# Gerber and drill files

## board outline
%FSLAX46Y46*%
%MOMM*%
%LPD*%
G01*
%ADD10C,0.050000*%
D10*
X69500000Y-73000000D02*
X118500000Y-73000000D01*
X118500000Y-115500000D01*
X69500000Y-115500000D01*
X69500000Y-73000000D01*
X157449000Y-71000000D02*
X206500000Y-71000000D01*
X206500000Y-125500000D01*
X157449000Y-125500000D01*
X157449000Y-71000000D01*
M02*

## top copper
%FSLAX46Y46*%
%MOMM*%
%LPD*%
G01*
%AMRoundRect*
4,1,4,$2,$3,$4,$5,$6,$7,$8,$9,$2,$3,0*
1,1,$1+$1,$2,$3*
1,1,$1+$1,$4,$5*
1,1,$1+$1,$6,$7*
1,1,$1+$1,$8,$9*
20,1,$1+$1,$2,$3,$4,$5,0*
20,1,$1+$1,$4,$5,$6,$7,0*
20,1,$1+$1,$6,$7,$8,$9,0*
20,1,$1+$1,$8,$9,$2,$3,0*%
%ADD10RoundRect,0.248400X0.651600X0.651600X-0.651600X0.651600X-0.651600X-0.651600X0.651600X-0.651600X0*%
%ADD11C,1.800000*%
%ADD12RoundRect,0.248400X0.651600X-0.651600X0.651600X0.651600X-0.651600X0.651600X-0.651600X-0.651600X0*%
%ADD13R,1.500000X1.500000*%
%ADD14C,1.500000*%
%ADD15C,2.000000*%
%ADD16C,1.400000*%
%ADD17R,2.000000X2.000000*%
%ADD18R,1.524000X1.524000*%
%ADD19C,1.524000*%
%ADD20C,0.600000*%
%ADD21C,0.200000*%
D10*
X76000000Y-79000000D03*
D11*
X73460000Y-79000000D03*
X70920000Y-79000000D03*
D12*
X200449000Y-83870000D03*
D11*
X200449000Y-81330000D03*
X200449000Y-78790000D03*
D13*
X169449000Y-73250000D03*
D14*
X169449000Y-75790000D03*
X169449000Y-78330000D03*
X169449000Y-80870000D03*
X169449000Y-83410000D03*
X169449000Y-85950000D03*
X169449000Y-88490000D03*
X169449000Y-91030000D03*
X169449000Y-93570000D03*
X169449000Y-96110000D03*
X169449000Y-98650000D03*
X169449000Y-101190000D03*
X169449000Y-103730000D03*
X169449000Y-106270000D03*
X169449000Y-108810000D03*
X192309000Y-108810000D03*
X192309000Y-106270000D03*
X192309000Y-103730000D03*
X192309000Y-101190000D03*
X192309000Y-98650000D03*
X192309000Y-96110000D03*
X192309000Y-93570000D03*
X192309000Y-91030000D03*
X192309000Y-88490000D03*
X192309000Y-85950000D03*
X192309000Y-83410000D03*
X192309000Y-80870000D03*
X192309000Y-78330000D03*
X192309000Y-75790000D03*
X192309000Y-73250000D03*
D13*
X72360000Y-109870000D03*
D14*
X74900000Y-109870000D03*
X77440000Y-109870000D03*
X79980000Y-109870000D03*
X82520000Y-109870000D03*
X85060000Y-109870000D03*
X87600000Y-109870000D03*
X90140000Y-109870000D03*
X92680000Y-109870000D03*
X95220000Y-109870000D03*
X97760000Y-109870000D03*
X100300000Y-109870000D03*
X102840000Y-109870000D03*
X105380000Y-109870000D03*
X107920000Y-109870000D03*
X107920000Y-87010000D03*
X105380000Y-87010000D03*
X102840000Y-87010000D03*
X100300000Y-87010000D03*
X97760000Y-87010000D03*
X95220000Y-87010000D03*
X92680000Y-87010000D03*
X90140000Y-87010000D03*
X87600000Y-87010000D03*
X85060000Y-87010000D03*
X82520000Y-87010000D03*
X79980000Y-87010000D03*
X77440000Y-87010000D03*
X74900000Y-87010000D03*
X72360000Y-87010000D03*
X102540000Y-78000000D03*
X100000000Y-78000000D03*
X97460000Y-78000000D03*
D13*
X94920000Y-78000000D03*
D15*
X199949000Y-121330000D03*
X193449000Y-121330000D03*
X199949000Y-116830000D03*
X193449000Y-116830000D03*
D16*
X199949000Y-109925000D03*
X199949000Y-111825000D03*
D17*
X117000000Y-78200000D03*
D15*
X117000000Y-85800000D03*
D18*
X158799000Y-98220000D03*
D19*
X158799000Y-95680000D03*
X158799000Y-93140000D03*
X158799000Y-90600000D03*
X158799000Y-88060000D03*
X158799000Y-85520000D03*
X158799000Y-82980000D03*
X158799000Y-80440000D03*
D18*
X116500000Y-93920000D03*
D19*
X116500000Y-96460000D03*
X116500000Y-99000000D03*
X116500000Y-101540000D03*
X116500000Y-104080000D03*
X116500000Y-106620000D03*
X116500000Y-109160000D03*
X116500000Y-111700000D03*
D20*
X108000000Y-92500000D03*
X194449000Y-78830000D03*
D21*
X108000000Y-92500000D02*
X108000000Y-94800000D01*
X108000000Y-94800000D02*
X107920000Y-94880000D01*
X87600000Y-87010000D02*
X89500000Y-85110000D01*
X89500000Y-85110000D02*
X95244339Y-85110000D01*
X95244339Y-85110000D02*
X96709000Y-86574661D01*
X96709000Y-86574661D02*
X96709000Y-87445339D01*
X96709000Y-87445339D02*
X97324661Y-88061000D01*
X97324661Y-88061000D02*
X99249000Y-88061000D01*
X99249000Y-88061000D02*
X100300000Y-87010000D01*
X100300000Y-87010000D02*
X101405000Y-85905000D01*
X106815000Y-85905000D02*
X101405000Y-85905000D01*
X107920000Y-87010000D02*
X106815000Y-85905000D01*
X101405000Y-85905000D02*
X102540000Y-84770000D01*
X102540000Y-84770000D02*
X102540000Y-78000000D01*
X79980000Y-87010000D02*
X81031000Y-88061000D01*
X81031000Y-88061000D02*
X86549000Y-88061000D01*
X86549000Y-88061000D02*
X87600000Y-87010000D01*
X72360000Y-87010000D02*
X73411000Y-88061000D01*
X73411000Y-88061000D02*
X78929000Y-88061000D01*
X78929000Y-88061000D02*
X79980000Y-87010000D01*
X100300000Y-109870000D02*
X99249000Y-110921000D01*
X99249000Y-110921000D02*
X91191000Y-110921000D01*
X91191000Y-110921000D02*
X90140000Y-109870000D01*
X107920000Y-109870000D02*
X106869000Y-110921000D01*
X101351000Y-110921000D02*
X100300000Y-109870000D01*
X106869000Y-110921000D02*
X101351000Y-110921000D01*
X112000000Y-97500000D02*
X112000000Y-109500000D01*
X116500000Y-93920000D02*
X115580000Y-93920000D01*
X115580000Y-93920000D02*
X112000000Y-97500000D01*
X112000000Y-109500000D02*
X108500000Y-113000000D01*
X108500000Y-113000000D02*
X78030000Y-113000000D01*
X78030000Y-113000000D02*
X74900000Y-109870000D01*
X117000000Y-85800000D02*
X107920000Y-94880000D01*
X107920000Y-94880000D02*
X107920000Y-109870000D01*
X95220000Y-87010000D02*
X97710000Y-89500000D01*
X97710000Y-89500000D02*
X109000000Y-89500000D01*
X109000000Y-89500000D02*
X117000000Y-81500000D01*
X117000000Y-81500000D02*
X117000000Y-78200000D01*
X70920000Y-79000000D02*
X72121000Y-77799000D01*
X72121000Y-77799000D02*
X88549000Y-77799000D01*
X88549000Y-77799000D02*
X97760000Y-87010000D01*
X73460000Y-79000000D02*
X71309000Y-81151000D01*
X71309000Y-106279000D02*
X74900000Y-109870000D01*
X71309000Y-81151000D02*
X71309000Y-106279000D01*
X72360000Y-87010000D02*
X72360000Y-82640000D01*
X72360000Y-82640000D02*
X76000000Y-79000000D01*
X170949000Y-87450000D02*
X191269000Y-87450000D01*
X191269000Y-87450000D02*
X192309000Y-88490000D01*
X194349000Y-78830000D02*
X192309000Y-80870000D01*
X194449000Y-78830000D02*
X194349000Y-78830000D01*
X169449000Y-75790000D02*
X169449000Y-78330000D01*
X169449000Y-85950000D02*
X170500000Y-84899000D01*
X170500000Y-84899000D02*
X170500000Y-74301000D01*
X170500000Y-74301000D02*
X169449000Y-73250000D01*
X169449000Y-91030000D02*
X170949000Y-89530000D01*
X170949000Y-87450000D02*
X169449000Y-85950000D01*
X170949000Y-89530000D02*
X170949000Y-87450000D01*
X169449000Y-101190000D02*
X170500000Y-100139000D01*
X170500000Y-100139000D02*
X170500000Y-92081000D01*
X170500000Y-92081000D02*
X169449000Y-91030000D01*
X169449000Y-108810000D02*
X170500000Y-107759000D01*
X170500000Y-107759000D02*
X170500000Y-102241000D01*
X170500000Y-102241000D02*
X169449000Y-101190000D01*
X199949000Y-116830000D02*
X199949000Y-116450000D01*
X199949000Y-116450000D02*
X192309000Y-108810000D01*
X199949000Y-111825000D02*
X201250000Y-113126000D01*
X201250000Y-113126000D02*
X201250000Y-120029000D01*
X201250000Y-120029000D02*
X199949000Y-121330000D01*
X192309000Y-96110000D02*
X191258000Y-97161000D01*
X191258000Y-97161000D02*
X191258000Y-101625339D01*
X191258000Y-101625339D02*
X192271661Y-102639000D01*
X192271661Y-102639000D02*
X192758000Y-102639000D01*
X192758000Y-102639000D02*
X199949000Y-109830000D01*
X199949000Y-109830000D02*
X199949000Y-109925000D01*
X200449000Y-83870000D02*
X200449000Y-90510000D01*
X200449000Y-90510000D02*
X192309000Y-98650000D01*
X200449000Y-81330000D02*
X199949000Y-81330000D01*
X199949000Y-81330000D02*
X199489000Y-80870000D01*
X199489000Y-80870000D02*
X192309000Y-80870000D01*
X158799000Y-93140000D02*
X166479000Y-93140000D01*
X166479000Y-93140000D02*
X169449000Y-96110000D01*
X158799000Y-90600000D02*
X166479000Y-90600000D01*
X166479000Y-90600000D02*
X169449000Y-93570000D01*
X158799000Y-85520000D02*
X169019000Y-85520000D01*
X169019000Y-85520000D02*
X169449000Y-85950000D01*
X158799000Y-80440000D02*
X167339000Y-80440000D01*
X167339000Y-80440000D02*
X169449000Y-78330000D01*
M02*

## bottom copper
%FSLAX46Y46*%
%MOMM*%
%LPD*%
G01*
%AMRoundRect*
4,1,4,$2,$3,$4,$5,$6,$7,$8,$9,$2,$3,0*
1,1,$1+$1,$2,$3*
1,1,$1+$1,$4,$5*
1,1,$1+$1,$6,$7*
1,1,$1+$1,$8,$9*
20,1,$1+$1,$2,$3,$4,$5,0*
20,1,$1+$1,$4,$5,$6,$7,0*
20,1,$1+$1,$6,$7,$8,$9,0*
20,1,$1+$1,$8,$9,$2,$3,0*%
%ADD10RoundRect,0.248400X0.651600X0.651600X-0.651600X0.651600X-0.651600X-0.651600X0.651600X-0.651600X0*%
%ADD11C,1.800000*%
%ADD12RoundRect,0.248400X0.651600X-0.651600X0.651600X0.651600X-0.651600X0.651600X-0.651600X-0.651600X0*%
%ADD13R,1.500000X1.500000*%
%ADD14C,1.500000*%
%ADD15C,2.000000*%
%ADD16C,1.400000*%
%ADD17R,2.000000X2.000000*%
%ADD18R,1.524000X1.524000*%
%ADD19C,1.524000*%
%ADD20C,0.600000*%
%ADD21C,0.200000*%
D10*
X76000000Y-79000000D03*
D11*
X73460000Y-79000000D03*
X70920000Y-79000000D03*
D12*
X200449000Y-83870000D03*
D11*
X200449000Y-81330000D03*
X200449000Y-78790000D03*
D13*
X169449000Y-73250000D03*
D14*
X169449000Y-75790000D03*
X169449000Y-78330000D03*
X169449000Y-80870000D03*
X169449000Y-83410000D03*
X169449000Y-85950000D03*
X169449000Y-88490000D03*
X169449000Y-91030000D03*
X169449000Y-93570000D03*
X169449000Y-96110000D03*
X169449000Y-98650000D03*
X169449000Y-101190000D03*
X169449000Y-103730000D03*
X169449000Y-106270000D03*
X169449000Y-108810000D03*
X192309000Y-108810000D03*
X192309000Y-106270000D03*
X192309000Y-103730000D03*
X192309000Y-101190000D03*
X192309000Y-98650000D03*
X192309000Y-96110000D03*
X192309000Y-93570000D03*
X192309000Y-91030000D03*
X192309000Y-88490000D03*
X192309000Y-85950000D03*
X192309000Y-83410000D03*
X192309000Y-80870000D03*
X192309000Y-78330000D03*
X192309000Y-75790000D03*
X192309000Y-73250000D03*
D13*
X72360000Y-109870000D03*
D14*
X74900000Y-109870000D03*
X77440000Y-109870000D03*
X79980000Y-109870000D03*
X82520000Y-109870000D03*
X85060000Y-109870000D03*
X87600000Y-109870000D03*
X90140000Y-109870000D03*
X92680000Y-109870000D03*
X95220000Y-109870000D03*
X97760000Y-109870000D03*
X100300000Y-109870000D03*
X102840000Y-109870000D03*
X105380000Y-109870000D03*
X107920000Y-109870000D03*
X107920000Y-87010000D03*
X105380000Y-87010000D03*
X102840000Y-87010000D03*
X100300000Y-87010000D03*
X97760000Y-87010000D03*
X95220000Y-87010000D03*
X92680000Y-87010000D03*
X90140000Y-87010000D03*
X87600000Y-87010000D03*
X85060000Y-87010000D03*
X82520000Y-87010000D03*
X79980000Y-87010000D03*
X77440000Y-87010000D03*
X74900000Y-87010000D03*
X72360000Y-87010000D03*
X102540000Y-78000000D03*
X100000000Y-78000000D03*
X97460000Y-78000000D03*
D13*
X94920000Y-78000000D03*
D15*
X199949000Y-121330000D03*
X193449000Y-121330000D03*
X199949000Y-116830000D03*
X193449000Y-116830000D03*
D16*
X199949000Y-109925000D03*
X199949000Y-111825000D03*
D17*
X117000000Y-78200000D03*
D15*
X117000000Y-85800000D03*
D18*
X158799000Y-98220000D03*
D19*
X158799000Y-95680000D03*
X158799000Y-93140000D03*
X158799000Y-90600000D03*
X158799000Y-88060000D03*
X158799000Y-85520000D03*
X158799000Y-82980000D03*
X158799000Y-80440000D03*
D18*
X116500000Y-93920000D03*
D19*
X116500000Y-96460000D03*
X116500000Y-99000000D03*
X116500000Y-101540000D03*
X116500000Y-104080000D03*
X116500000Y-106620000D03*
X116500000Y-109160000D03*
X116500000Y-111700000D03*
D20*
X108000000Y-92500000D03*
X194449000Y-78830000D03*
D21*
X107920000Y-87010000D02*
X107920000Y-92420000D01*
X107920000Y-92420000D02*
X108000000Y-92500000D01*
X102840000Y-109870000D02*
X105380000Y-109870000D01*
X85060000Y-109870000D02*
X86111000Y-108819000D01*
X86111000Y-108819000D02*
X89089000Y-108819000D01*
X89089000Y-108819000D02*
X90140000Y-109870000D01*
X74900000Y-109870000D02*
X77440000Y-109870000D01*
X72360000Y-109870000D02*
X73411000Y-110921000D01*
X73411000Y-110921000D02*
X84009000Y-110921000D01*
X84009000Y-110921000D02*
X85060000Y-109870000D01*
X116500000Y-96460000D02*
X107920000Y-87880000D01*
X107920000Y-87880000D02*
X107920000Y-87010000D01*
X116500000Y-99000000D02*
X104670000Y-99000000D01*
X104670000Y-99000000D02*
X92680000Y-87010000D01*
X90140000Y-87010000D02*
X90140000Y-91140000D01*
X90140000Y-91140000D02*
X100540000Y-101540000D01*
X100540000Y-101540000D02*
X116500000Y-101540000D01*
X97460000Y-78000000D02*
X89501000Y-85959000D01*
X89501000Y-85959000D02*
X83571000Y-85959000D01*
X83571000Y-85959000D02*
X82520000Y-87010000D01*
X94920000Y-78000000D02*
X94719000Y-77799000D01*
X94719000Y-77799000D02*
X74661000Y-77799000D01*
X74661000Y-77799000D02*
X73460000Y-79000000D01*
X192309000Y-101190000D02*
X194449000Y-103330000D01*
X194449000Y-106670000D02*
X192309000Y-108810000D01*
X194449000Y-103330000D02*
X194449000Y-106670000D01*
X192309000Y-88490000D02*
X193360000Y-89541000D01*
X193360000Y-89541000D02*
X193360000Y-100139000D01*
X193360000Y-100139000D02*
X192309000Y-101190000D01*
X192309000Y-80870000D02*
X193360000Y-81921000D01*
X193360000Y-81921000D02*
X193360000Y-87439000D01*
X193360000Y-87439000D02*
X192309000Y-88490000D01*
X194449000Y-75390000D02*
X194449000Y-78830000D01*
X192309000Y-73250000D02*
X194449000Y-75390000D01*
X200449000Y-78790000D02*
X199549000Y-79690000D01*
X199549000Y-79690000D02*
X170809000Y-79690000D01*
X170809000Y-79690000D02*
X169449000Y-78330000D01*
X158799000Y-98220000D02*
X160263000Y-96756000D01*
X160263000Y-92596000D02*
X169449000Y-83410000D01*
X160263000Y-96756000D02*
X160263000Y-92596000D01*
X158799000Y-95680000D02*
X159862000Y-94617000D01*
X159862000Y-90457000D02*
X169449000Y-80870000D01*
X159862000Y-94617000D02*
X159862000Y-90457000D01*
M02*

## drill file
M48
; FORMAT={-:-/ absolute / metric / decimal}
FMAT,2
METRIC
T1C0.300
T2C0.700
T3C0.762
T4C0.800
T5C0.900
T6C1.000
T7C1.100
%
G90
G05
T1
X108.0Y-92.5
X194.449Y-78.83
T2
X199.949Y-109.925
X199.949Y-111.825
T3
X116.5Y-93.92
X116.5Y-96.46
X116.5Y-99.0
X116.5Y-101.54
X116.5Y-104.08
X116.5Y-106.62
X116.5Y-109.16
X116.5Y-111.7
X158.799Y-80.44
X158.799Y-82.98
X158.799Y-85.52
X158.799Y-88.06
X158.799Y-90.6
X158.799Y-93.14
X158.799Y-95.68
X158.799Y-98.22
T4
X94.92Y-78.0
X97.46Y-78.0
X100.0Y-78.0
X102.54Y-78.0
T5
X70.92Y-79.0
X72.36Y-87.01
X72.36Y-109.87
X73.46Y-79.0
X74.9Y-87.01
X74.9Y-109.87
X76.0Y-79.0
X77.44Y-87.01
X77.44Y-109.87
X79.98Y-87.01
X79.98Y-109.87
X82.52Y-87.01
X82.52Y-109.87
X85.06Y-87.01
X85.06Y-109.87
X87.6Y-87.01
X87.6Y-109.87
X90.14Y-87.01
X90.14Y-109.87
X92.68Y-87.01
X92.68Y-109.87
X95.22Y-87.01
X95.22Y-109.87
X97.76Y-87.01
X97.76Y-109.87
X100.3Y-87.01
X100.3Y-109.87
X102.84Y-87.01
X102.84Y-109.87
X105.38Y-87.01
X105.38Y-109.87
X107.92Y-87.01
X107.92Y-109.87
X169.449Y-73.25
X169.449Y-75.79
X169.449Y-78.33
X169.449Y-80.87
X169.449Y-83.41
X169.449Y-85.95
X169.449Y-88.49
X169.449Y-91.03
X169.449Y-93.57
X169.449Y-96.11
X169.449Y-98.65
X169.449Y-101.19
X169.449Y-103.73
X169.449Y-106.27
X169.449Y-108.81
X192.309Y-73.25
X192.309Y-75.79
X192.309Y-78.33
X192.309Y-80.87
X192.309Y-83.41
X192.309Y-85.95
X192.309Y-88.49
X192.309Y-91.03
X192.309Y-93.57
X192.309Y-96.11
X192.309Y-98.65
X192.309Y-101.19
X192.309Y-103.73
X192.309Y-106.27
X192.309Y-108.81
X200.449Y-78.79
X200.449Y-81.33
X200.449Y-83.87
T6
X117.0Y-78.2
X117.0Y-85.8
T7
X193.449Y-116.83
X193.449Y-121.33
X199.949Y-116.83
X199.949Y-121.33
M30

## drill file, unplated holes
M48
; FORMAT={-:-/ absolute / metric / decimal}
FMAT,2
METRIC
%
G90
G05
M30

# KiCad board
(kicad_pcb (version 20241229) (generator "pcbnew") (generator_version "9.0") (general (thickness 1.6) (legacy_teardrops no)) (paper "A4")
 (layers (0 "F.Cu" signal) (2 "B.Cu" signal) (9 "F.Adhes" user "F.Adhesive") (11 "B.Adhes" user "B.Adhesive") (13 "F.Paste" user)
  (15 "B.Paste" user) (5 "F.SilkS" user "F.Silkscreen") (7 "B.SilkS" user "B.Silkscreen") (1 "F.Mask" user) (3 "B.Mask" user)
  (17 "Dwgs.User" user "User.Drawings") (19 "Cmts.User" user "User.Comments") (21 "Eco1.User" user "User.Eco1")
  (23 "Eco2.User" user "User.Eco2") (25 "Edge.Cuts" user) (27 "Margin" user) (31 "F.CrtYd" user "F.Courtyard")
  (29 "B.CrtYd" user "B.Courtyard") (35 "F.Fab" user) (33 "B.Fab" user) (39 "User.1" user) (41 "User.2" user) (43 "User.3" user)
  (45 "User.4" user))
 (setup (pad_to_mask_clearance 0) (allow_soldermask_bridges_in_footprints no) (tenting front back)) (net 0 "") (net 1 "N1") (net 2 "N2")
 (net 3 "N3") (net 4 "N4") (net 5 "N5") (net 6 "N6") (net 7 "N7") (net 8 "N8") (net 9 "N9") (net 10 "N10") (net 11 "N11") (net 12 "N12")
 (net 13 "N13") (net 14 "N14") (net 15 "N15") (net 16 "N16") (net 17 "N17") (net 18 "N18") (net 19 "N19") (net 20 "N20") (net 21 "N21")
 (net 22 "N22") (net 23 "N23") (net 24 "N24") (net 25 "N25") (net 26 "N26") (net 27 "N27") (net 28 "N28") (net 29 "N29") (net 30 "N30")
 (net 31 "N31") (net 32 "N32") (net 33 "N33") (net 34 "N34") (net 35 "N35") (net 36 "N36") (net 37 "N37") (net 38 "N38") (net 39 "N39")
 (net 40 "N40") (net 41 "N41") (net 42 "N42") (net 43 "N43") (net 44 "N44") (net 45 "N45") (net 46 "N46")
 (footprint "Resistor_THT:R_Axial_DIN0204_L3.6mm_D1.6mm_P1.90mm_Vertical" (layer "F.Cu") (at 199.949 109.925 -90)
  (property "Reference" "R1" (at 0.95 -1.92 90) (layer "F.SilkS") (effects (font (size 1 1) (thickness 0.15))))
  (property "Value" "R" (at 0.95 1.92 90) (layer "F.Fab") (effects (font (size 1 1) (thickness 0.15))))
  (pad "1" thru_hole circle (at 0 0 270) (size 1.4 1.4) (drill 0.7) (layers "*.Cu" "*.Mask") (remove_unused_layers no) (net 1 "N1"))
  (pad "2" thru_hole circle (at 1.9 0 270) (size 1.4 1.4) (drill 0.7) (layers "*.Cu" "*.Mask") (remove_unused_layers no) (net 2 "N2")))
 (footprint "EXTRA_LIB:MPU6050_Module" (layer "F.Cu") (at 116.5 93.92)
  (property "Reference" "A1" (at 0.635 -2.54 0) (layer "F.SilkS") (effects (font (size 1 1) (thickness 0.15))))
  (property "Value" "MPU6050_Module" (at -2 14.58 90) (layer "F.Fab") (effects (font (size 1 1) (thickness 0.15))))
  (pad "1" thru_hole rect (at 0 0) (size 1.524 1.524) (drill 0.762) (layers "*.Cu" "*.Mask") (remove_unused_layers no) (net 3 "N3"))
  (pad "2" thru_hole circle (at 0 2.54) (size 1.524 1.524) (drill 0.762) (layers "*.Cu" "*.Mask") (remove_unused_layers no) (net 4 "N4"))
  (pad "3" thru_hole circle (at 0 5.08) (size 1.524 1.524) (drill 0.762) (layers "*.Cu" "*.Mask") (remove_unused_layers no) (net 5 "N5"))
  (pad "4" thru_hole circle (at 0 7.62) (size 1.524 1.524) (drill 0.762) (layers "*.Cu" "*.Mask") (remove_unused_layers no) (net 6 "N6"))
  (pad "5" thru_hole circle (at 0 10.16) (size 1.524 1.524) (drill 0.762) (layers "*.Cu" "*.Mask") (remove_unused_layers no) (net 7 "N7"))
  (pad "6" thru_hole circle (at 0 12.7) (size 1.524 1.524) (drill 0.762) (layers "*.Cu" "*.Mask") (remove_unused_layers no) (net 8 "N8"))
  (pad "7" thru_hole circle (at 0 15.24) (size 1.524 1.524) (drill 0.762) (layers "*.Cu" "*.Mask") (remove_unused_layers no) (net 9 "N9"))
  (pad "8" thru_hole circle (at 0 17.78) (size 1.524 1.524) (drill 0.762) (layers "*.Cu" "*.Mask") (remove_unused_layers no) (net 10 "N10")))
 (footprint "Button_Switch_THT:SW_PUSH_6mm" (layer "F.Cu") (at 199.949 121.33 180)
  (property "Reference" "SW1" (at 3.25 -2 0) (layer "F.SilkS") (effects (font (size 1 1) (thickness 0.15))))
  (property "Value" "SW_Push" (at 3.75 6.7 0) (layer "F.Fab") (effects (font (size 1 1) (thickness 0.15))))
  (pad "1" thru_hole circle (at 0 0 270) (size 2 2) (drill 1.1) (layers "*.Cu" "*.Mask") (remove_unused_layers no) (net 2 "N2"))
  (pad "1" thru_hole circle (at 6.5 0 270) (size 2 2) (drill 1.1) (layers "*.Cu" "*.Mask") (remove_unused_layers no) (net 2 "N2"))
  (pad "2" thru_hole circle (at 0 4.5 270) (size 2 2) (drill 1.1) (layers "*.Cu" "*.Mask") (remove_unused_layers no) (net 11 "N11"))
  (pad "2" thru_hole circle (at 6.5 4.5 270) (size 2 2) (drill 1.1) (layers "*.Cu" "*.Mask") (remove_unused_layers no) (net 11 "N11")))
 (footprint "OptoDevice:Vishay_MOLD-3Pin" (layer "F.Cu") (at 200.449 83.87 90)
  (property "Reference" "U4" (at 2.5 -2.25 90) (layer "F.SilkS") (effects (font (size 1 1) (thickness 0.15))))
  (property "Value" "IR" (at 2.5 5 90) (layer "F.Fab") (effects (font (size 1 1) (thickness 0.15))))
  (pad "1" thru_hole roundrect (at 0 0 90) (size 1.8 1.8) (drill 0.9) (layers "*.Cu" "*.Mask") (remove_unused_layers no)
   (roundrect_rratio 0.138) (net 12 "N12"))
  (pad "2" thru_hole circle (at 2.54 0 90) (size 1.8 1.8) (drill 0.9) (layers "*.Cu" "*.Mask") (remove_unused_layers no) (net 11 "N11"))
  (pad "3" thru_hole circle (at 5.08 0 90) (size 1.8 1.8) (drill 0.9) (layers "*.Cu" "*.Mask") (remove_unused_layers no) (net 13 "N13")))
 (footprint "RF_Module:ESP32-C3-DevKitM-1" (layer "F.Cu") (at 72.36 109.87 90)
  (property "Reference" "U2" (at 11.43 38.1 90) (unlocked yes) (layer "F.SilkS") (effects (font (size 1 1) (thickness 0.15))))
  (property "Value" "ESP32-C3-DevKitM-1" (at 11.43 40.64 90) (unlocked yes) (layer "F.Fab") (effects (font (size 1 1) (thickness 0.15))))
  (pad "1" thru_hole rect (at 0 0 90) (size 1.5 1.5) (drill 0.9) (layers "*.Cu" "*.Mask") (remove_unused_layers yes) (keep_end_layers yes)
   (zone_layer_connections) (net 4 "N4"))
  (pad "2" thru_hole circle (at 0 2.54 90) (size 1.5 1.5) (drill 0.9) (layers "*.Cu" "*.Mask") (remove_unused_layers yes)
   (keep_end_layers yes) (zone_layer_connections) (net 3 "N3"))
  (pad "3" thru_hole circle (at 0 5.08 90) (size 1.5 1.5) (drill 0.9) (layers "*.Cu" "*.Mask") (remove_unused_layers yes)
   (keep_end_layers yes) (zone_layer_connections) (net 3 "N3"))
  (pad "4" thru_hole circle (at 0 7.62 90) (size 1.5 1.5) (drill 0.9) (layers "*.Cu" "*.Mask") (remove_unused_layers yes)
   (keep_end_layers yes) (zone_layer_connections) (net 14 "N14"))
  (pad "5" thru_hole circle (at 0 10.16 90) (size 1.5 1.5) (drill 0.9) (layers "*.Cu" "*.Mask") (remove_unused_layers yes)
   (keep_end_layers yes) (zone_layer_connections) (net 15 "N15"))
  (pad "6" thru_hole circle (at 0 12.7 90) (size 1.5 1.5) (drill 0.9) (layers "*.Cu" "*.Mask") (remove_unused_layers yes)
   (keep_end_layers yes) (zone_layer_connections) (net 4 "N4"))
  (pad "7" thru_hole circle (at 0 15.24 90) (size 1.5 1.5) (drill 0.9) (layers "*.Cu" "*.Mask") (remove_unused_layers yes)
   (keep_end_layers yes) (zone_layer_connections) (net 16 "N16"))
  (pad "8" thru_hole circle (at 0 17.78 90) (size 1.5 1.5) (drill 0.9) (layers "*.Cu" "*.Mask") (remove_unused_layers yes)
   (keep_end_layers yes) (zone_layer_connections) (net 4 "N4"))
  (pad "9" thru_hole circle (at 0 20.32 90) (size 1.5 1.5) (drill 0.9) (layers "*.Cu" "*.Mask") (remove_unused_layers yes)
   (keep_end_layers yes) (zone_layer_connections) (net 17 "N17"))
  (pad "10" thru_hole circle (at 0 22.86 90) (size 1.5 1.5) (drill 0.9) (layers "*.Cu" "*.Mask") (remove_unused_layers yes)
   (keep_end_layers yes) (zone_layer_connections) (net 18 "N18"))
  (pad "11" thru_hole circle (at 0 25.4 90) (size 1.5 1.5) (drill 0.9) (layers "*.Cu" "*.Mask") (remove_unused_layers yes)
   (keep_end_layers yes) (zone_layer_connections) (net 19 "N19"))
  (pad "12" thru_hole circle (at 0 27.94 90) (size 1.5 1.5) (drill 0.9) (layers "*.Cu" "*.Mask") (remove_unused_layers yes)
   (keep_end_layers yes) (zone_layer_connections) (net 4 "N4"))
  (pad "13" thru_hole circle (at 0 30.48 90) (size 1.5 1.5) (drill 0.9) (layers "*.Cu" "*.Mask") (remove_unused_layers yes)
   (keep_end_layers yes) (zone_layer_connections) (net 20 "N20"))
  (pad "14" thru_hole circle (at 0 33.02 90) (size 1.5 1.5) (drill 0.9) (layers "*.Cu" "*.Mask") (remove_unused_layers yes)
   (keep_end_layers yes) (zone_layer_connections) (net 20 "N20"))
  (pad "15" thru_hole circle (at 0 35.56 90) (size 1.5 1.5) (drill 0.9) (layers "*.Cu" "*.Mask") (remove_unused_layers yes)
   (keep_end_layers yes) (zone_layer_connections) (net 4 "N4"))
  (pad "16" thru_hole circle (at 22.86 35.56 90) (size 1.5 1.5) (drill 0.9) (layers "*.Cu" "*.Mask") (remove_unused_layers yes)
   (keep_end_layers yes) (zone_layer_connections) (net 4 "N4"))
  (pad "17" thru_hole circle (at 22.86 33.02 90) (size 1.5 1.5) (drill 0.9) (layers "*.Cu" "*.Mask") (remove_unused_layers yes)
   (keep_end_layers yes) (zone_layer_connections) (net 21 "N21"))
  (pad "18" thru_hole circle (at 22.86 30.48 90) (size 1.5 1.5) (drill 0.9) (layers "*.Cu" "*.Mask") (remove_unused_layers yes)
   (keep_end_layers yes) (zone_layer_connections) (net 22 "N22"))
  (pad "19" thru_hole circle (at 22.86 27.94 90) (size 1.5 1.5) (drill 0.9) (layers "*.Cu" "*.Mask") (remove_unused_layers yes)
   (keep_end_layers yes) (zone_layer_connections) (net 4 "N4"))
  (pad "20" thru_hole circle (at 22.86 25.4 90) (size 1.5 1.5) (drill 0.9) (layers "*.Cu" "*.Mask") (remove_unused_layers yes)
   (keep_end_layers yes) (zone_layer_connections) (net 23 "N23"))
  (pad "21" thru_hole circle (at 22.86 22.86 90) (size 1.5 1.5) (drill 0.9) (layers "*.Cu" "*.Mask") (remove_unused_layers yes)
   (keep_end_layers yes) (zone_layer_connections) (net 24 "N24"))
  (pad "22" thru_hole circle (at 22.86 20.32 90) (size 1.5 1.5) (drill 0.9) (layers "*.Cu" "*.Mask") (remove_unused_layers yes)
   (keep_end_layers yes) (zone_layer_connections) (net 5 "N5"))
  (pad "23" thru_hole circle (at 22.86 17.78 90) (size 1.5 1.5) (drill 0.9) (layers "*.Cu" "*.Mask") (remove_unused_layers yes)
   (keep_end_layers yes) (zone_layer_connections) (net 6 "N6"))
  (pad "24" thru_hole circle (at 22.86 15.24 90) (size 1.5 1.5) (drill 0.9) (layers "*.Cu" "*.Mask") (remove_unused_layers yes)
   (keep_end_layers yes) (zone_layer_connections) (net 4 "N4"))
  (pad "25" thru_hole circle (at 22.86 12.7 90) (size 1.5 1.5) (drill 0.9) (layers "*.Cu" "*.Mask") (remove_unused_layers yes)
   (keep_end_layers yes) (zone_layer_connections) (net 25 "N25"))
  (pad "26" thru_hole circle (at 22.86 10.16 90) (size 1.5 1.5) (drill 0.9) (layers "*.Cu" "*.Mask") (remove_unused_layers yes)
   (keep_end_layers yes) (zone_layer_connections) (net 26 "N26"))
  (pad "27" thru_hole circle (at 22.86 7.62 90) (size 1.5 1.5) (drill 0.9) (layers "*.Cu" "*.Mask") (remove_unused_layers yes)
   (keep_end_layers yes) (zone_layer_connections) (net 4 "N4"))
  (pad "28" thru_hole circle (at 22.86 5.08 90) (size 1.5 1.5) (drill 0.9) (layers "*.Cu" "*.Mask") (remove_unused_layers yes)
   (keep_end_layers yes) (zone_layer_connections) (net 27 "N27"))
  (pad "29" thru_hole circle (at 22.86 2.54 90) (size 1.5 1.5) (drill 0.9) (layers "*.Cu" "*.Mask") (remove_unused_layers yes)
   (keep_end_layers yes) (zone_layer_connections) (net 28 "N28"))
  (pad "30" thru_hole circle (at 22.86 0 90) (size 1.5 1.5) (drill 0.9) (layers "*.Cu" "*.Mask") (remove_unused_layers yes)
   (keep_end_layers yes) (zone_layer_connections) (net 4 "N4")))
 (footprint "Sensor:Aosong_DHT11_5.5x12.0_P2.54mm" (layer "F.Cu") (at 94.92 78 90)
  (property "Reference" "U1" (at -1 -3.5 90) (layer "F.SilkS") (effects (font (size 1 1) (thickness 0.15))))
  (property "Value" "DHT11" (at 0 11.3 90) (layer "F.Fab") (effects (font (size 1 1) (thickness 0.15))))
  (pad "1" thru_hole rect (at 0 0 90) (size 1.5 1.5) (drill 0.8) (layers "*.Cu" "*.Mask") (remove_unused_layers no) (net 3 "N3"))
  (pad "2" thru_hole circle (at 0 2.54 90) (size 1.5 1.5) (drill 0.8) (layers "*.Cu" "*.Mask") (remove_unused_layers no) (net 26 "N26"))
  (pad "3" thru_hole circle (at 0 5.08 90) (size 1.5 1.5) (drill 0.8) (layers "*.Cu" "*.Mask") (remove_unused_layers no) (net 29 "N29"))
  (pad "4" thru_hole circle (at 0 7.62 90) (size 1.5 1.5) (drill 0.8) (layers "*.Cu" "*.Mask") (remove_unused_layers no) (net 4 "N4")))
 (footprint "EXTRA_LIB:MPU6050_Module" (layer "F.Cu") (at 158.799 98.22 180)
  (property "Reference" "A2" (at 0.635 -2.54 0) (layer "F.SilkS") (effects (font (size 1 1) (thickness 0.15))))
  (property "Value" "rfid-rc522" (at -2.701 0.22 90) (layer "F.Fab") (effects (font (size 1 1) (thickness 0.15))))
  (pad "1" thru_hole rect (at 0 0 180) (size 1.524 1.524) (drill 0.762) (layers "*.Cu" "*.Mask") (remove_unused_layers no) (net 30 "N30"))
  (pad "2" thru_hole circle (at 0 2.54 180) (size 1.524 1.524) (drill 0.762) (layers "*.Cu" "*.Mask") (remove_unused_layers no)
   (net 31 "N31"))
  (pad "3" thru_hole circle (at 0 5.08 180) (size 1.524 1.524) (drill 0.762) (layers "*.Cu" "*.Mask") (remove_unused_layers no)
   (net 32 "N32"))
  (pad "4" thru_hole circle (at 0 7.62 180) (size 1.524 1.524) (drill 0.762) (layers "*.Cu" "*.Mask") (remove_unused_layers no)
   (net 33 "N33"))
  (pad "5" thru_hole circle (at 0 10.16 180) (size 1.524 1.524) (drill 0.762) (layers "*.Cu" "*.Mask") (remove_unused_layers no)
   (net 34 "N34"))
  (pad "6" thru_hole circle (at 0 12.7 180) (size 1.524 1.524) (drill 0.762) (layers "*.Cu" "*.Mask") (remove_unused_layers no)
   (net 11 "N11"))
  (pad "7" thru_hole circle (at 0 15.24 180) (size 1.524 1.524) (drill 0.762) (layers "*.Cu" "*.Mask") (remove_unused_layers no)
   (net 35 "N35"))
  (pad "8" thru_hole circle (at 0 17.78 180) (size 1.524 1.524) (drill 0.762) (layers "*.Cu" "*.Mask") (remove_unused_layers no)
   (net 13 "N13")))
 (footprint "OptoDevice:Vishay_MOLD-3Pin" (layer "F.Cu") (at 76 79 180)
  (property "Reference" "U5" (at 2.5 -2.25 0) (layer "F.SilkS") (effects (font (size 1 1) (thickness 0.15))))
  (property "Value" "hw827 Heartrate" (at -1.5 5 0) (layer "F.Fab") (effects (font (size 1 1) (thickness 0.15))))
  (pad "1" thru_hole roundrect (at 0 0 180) (size 1.8 1.8) (drill 0.9) (layers "*.Cu" "*.Mask") (remove_unused_layers no)
   (roundrect_rratio 0.138) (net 4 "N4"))
  (pad "2" thru_hole circle (at 2.54 0 180) (size 1.8 1.8) (drill 0.9) (layers "*.Cu" "*.Mask") (remove_unused_layers no) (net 3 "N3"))
  (pad "3" thru_hole circle (at 5.08 0 180) (size 1.8 1.8) (drill 0.9) (layers "*.Cu" "*.Mask") (remove_unused_layers no) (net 23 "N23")))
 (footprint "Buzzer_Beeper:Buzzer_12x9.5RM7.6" (layer "F.Cu") (at 117 78.2 -90)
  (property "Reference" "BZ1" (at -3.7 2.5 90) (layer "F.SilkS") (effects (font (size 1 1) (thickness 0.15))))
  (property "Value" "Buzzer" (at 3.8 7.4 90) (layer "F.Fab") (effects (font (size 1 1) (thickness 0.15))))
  (pad "1" thru_hole rect (at 0 0 270) (size 2 2) (drill 1) (layers "*.Cu" "*.Mask") (remove_unused_layers no) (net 24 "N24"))
  (pad "2" thru_hole circle (at 7.6 0 270) (size 2 2) (drill 1) (layers "*.Cu" "*.Mask") (remove_unused_layers no) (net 4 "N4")))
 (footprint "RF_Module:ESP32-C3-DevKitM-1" (layer "F.Cu") (at 169.449 73.25)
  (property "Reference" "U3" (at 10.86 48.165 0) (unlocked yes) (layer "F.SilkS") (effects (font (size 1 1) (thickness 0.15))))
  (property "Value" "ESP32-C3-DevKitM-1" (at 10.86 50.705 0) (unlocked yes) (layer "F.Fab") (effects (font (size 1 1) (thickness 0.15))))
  (pad "1" thru_hole rect (at 0 0) (size 1.5 1.5) (drill 0.9) (layers "*.Cu" "*.Mask") (remove_unused_layers yes) (keep_end_layers yes)
   (zone_layer_connections) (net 11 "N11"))
  (pad "2" thru_hole circle (at 0 2.54) (size 1.5 1.5) (drill 0.9) (layers "*.Cu" "*.Mask") (remove_unused_layers yes) (keep_end_layers yes)
   (zone_layer_connections) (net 13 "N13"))
  (pad "3" thru_hole circle (at 0 5.08) (size 1.5 1.5) (drill 0.9) (layers "*.Cu" "*.Mask") (remove_unused_layers yes) (keep_end_layers yes)
   (zone_layer_connections) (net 13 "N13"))
  (pad "4" thru_hole circle (at 0 7.62) (size 1.5 1.5) (drill 0.9) (layers "*.Cu" "*.Mask") (remove_unused_layers yes) (keep_end_layers yes)
   (zone_layer_connections) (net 31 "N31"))
  (pad "5" thru_hole circle (at 0 10.16) (size 1.5 1.5) (drill 0.9) (layers "*.Cu" "*.Mask") (remove_unused_layers yes)
   (keep_end_layers yes) (zone_layer_connections) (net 30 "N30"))
  (pad "6" thru_hole circle (at 0 12.7) (size 1.5 1.5) (drill 0.9) (layers "*.Cu" "*.Mask") (remove_unused_layers yes) (keep_end_layers yes)
   (zone_layer_connections) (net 11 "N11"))
  (pad "7" thru_hole circle (at 0 15.24) (size 1.5 1.5) (drill 0.9) (layers "*.Cu" "*.Mask") (remove_unused_layers yes)
   (keep_end_layers yes) (zone_layer_connections) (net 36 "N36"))
  (pad "8" thru_hole circle (at 0 17.78) (size 1.5 1.5) (drill 0.9) (layers "*.Cu" "*.Mask") (remove_unused_layers yes)
   (keep_end_layers yes) (zone_layer_connections) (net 11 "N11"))
  (pad "9" thru_hole circle (at 0 20.32) (size 1.5 1.5) (drill 0.9) (layers "*.Cu" "*.Mask") (remove_unused_layers yes)
   (keep_end_layers yes) (zone_layer_connections) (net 33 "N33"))
  (pad "10" thru_hole circle (at 0 22.86) (size 1.5 1.5) (drill 0.9) (layers "*.Cu" "*.Mask") (remove_unused_layers yes)
   (keep_end_layers yes) (zone_layer_connections) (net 32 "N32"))
  (pad "11" thru_hole circle (at 0 25.4) (size 1.5 1.5) (drill 0.9) (layers "*.Cu" "*.Mask") (remove_unused_layers yes)
   (keep_end_layers yes) (zone_layer_connections) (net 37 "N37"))
  (pad "12" thru_hole circle (at 0 27.94) (size 1.5 1.5) (drill 0.9) (layers "*.Cu" "*.Mask") (remove_unused_layers yes)
   (keep_end_layers yes) (zone_layer_connections) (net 11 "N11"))
  (pad "13" thru_hole circle (at 0 30.48) (size 1.5 1.5) (drill 0.9) (layers "*.Cu" "*.Mask") (remove_unused_layers yes)
   (keep_end_layers yes) (zone_layer_connections) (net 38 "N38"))
  (pad "14" thru_hole circle (at 0 33.02) (size 1.5 1.5) (drill 0.9) (layers "*.Cu" "*.Mask") (remove_unused_layers yes)
   (keep_end_layers yes) (zone_layer_connections) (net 38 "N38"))
  (pad "15" thru_hole circle (at 0 35.56) (size 1.5 1.5) (drill 0.9) (layers "*.Cu" "*.Mask") (remove_unused_layers yes)
   (keep_end_layers yes) (zone_layer_connections) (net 11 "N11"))
  (pad "16" thru_hole circle (at 22.86 35.56) (size 1.5 1.5) (drill 0.9) (layers "*.Cu" "*.Mask") (remove_unused_layers yes)
   (keep_end_layers yes) (zone_layer_connections) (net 11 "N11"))
  (pad "17" thru_hole circle (at 22.86 33.02) (size 1.5 1.5) (drill 0.9) (layers "*.Cu" "*.Mask") (remove_unused_layers yes)
   (keep_end_layers yes) (zone_layer_connections) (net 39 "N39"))
  (pad "18" thru_hole circle (at 22.86 30.48) (size 1.5 1.5) (drill 0.9) (layers "*.Cu" "*.Mask") (remove_unused_layers yes)
   (keep_end_layers yes) (zone_layer_connections) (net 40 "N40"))
  (pad "19" thru_hole circle (at 22.86 27.94) (size 1.5 1.5) (drill 0.9) (layers "*.Cu" "*.Mask") (remove_unused_layers yes)
   (keep_end_layers yes) (zone_layer_connections) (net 11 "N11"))
  (pad "20" thru_hole circle (at 22.86 25.4) (size 1.5 1.5) (drill 0.9) (layers "*.Cu" "*.Mask") (remove_unused_layers yes)
   (keep_end_layers yes) (zone_layer_connections) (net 12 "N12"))
  (pad "21" thru_hole circle (at 22.86 22.86) (size 1.5 1.5) (drill 0.9) (layers "*.Cu" "*.Mask") (remove_unused_layers yes)
   (keep_end_layers yes) (zone_layer_connections) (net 1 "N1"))
  (pad "22" thru_hole circle (at 22.86 20.32) (size 1.5 1.5) (drill 0.9) (layers "*.Cu" "*.Mask") (remove_unused_layers yes)
   (keep_end_layers yes) (zone_layer_connections) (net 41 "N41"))
  (pad "23" thru_hole circle (at 22.86 17.78) (size 1.5 1.5) (drill 0.9) (layers "*.Cu" "*.Mask") (remove_unused_layers yes)
   (keep_end_layers yes) (zone_layer_connections) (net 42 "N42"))
  (pad "24" thru_hole circle (at 22.86 15.24) (size 1.5 1.5) (drill 0.9) (layers "*.Cu" "*.Mask") (remove_unused_layers yes)
   (keep_end_layers yes) (zone_layer_connections) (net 11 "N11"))
  (pad "25" thru_hole circle (at 22.86 12.7) (size 1.5 1.5) (drill 0.9) (layers "*.Cu" "*.Mask") (remove_unused_layers yes)
   (keep_end_layers yes) (zone_layer_connections) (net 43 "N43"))
  (pad "26" thru_hole circle (at 22.86 10.16) (size 1.5 1.5) (drill 0.9) (layers "*.Cu" "*.Mask") (remove_unused_layers yes)
   (keep_end_layers yes) (zone_layer_connections) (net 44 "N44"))
  (pad "27" thru_hole circle (at 22.86 7.62) (size 1.5 1.5) (drill 0.9) (layers "*.Cu" "*.Mask") (remove_unused_layers yes)
   (keep_end_layers yes) (zone_layer_connections) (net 11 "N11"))
  (pad "28" thru_hole circle (at 22.86 5.08) (size 1.5 1.5) (drill 0.9) (layers "*.Cu" "*.Mask") (remove_unused_layers yes)
   (keep_end_layers yes) (zone_layer_connections) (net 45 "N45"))
  (pad "29" thru_hole circle (at 22.86 2.54) (size 1.5 1.5) (drill 0.9) (layers "*.Cu" "*.Mask") (remove_unused_layers yes)
   (keep_end_layers yes) (zone_layer_connections) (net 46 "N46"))
  (pad "30" thru_hole circle (at 22.86 0) (size 1.5 1.5) (drill 0.9) (layers "*.Cu" "*.Mask") (remove_unused_layers yes)
   (keep_end_layers yes) (zone_layer_connections) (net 11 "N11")))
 (gr_rect (start 69.5 73) (end 118.5 115.5) (stroke (width 0.05) (type default)) (fill no) (layer "Edge.Cuts"))
 (gr_rect (start 157.449 71) (end 206.5 125.5) (stroke (width 0.05) (type default)) (fill no) (layer "Edge.Cuts"))
 (segment (start 71.309 106.279) (end 74.9 109.87) (width 0.2) (layer "F.Cu") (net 3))
 (segment (start 112 109.5) (end 108.5 113) (width 0.2) (layer "F.Cu") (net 3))
 (segment (start 116.5 93.92) (end 115.58 93.92) (width 0.2) (layer "F.Cu") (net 3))
 (segment (start 112 97.5) (end 112 109.5) (width 0.2) (layer "F.Cu") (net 3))
 (segment (start 115.58 93.92) (end 112 97.5) (width 0.2) (layer "F.Cu") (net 3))
 (segment (start 73.46 79) (end 71.309 81.151) (width 0.2) (layer "F.Cu") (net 3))
 (segment (start 108.5 113) (end 78.03 113) (width 0.2) (layer "F.Cu") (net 3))
 (segment (start 71.309 81.151) (end 71.309 106.279) (width 0.2) (layer "F.Cu") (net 3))
 (segment (start 78.03 113) (end 74.9 109.87) (width 0.2) (layer "F.Cu") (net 3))
 (segment (start 94.92 78) (end 94.719 77.799) (width 0.2) (layer "B.Cu") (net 3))
 (segment (start 94.719 77.799) (end 74.661 77.799) (width 0.2) (layer "B.Cu") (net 3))
 (segment (start 74.661 77.799) (end 73.46 79) (width 0.2) (layer "B.Cu") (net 3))
 (segment (start 74.9 109.87) (end 77.44 109.87) (width 0.2) (layer "B.Cu") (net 3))
 (segment (start 90.14 91.14) (end 100.54 101.54) (width 0.2) (layer "B.Cu") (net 6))
 (segment (start 100.54 101.54) (end 116.5 101.54) (width 0.2) (layer "B.Cu") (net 6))
 (segment (start 90.14 87.01) (end 90.14 91.14) (width 0.2) (layer "B.Cu") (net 6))
 (segment (start 73.411 88.061) (end 78.929 88.061) (width 0.2) (layer "F.Cu") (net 4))
 (segment (start 99.249 88.061) (end 100.3 87.01) (width 0.2) (layer "F.Cu") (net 4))
 (segment (start 72.36 87.01) (end 72.36 82.64) (width 0.2) (layer "F.Cu") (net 4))
 (segment (start 107.92 87.01) (end 106.815 85.905) (width 0.2) (layer "F.Cu") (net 4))
 (segment (start 96.709 87.445339) (end 97.324661 88.061) (width 0.2) (layer "F.Cu") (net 4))
 (segment (start 72.36 82.64) (end 76 79) (width 0.2) (layer "F.Cu") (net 4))
 (segment (start 107.92 109.87) (end 106.869 110.921) (width 0.2) (layer "F.Cu") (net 4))
 (segment (start 100.3 87.01) (end 101.405 85.905) (width 0.2) (layer "F.Cu") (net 4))
 (segment (start 97.324661 88.061) (end 99.249 88.061) (width 0.2) (layer "F.Cu") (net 4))
 (segment (start 81.031 88.061) (end 86.549 88.061) (width 0.2) (layer "F.Cu") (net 4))
 (segment (start 96.709 86.574661) (end 96.709 87.445339) (width 0.2) (layer "F.Cu") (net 4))
 (segment (start 106.869 110.921) (end 101.351 110.921) (width 0.2) (layer "F.Cu") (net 4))
 (segment (start 108 94.8) (end 107.92 94.88) (width 0.2) (layer "F.Cu") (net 4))
 (segment (start 101.351 110.921) (end 100.3 109.87) (width 0.2) (layer "F.Cu") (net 4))
 (segment (start 101.405 85.905) (end 102.54 84.77) (width 0.2) (layer "F.Cu") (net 4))
 (segment (start 72.36 87.01) (end 73.411 88.061) (width 0.2) (layer "F.Cu") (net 4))
 (segment (start 106.815 85.905) (end 101.405 85.905) (width 0.2) (layer "F.Cu") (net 4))
 (segment (start 117 85.8) (end 107.92 94.88) (width 0.2) (layer "F.Cu") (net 4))
 (segment (start 78.929 88.061) (end 79.98 87.01) (width 0.2) (layer "F.Cu") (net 4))
 (segment (start 79.98 87.01) (end 81.031 88.061) (width 0.2) (layer "F.Cu") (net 4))
 (segment (start 86.549 88.061) (end 87.6 87.01) (width 0.2) (layer "F.Cu") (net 4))
 (segment (start 89.5 85.11) (end 95.244339 85.11) (width 0.2) (layer "F.Cu") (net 4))
 (segment (start 99.249 110.921) (end 91.191 110.921) (width 0.2) (layer "F.Cu") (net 4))
 (segment (start 87.6 87.01) (end 89.5 85.11) (width 0.2) (layer "F.Cu") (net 4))
 (segment (start 91.191 110.921) (end 90.14 109.87) (width 0.2) (layer "F.Cu") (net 4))
 (segment (start 95.244339 85.11) (end 96.709 86.574661) (width 0.2) (layer "F.Cu") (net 4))
 (segment (start 108 92.5) (end 108 94.8) (width 0.2) (layer "F.Cu") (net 4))
 (segment (start 102.54 84.77) (end 102.54 78) (width 0.2) (layer "F.Cu") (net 4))
 (segment (start 107.92 94.88) (end 107.92 109.87) (width 0.2) (layer "F.Cu") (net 4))
 (segment (start 100.3 109.87) (end 99.249 110.921) (width 0.2) (layer "F.Cu") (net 4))
 (via (at 108 92.5) (size 0.6) (drill 0.3) (layers "F.Cu" "B.Cu") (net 4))
 (segment (start 84.009 110.921) (end 85.06 109.87) (width 0.2) (layer "B.Cu") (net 4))
 (segment (start 72.36 109.87) (end 73.411 110.921) (width 0.2) (layer "B.Cu") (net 4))
 (segment (start 107.92 92.42) (end 108 92.5) (width 0.2) (layer "B.Cu") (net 4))
 (segment (start 107.92 87.01) (end 107.92 92.42) (width 0.2) (layer "B.Cu") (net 4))
 (segment (start 86.111 108.819) (end 89.089 108.819) (width 0.2) (layer "B.Cu") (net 4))
 (segment (start 73.411 110.921) (end 84.009 110.921) (width 0.2) (layer "B.Cu") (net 4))
 (segment (start 116.5 96.46) (end 107.92 87.88) (width 0.2) (layer "B.Cu") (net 4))
 (segment (start 85.06 109.87) (end 86.111 108.819) (width 0.2) (layer "B.Cu") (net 4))
 (segment (start 89.089 108.819) (end 90.14 109.87) (width 0.2) (layer "B.Cu") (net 4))
 (segment (start 107.92 87.88) (end 107.92 87.01) (width 0.2) (layer "B.Cu") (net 4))
 (segment (start 104.67 99) (end 92.68 87.01) (width 0.2) (layer "B.Cu") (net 5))
 (segment (start 116.5 99) (end 104.67 99) (width 0.2) (layer "B.Cu") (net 5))
 (segment (start 158.799 98.22) (end 160.263 96.756) (width 0.2) (layer "B.Cu") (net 30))
 (segment (start 160.263 92.596) (end 169.449 83.41) (width 0.2) (layer "B.Cu") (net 30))
 (segment (start 160.263 96.756) (end 160.263 92.596) (width 0.2) (layer "B.Cu") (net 30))
 (segment (start 159.862 94.617) (end 159.862 90.457) (width 0.2) (layer "B.Cu") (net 31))
 (segment (start 158.799 95.68) (end 159.862 94.617) (width 0.2) (layer "B.Cu") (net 31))
 (segment (start 159.862 90.457) (end 169.449 80.87) (width 0.2) (layer "B.Cu") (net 31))
 (segment (start 166.479 93.14) (end 169.449 96.11) (width 0.2) (layer "F.Cu") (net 32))
 (segment (start 158.799 93.14) (end 166.479 93.14) (width 0.2) (layer "F.Cu") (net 32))
 (segment (start 191.269 87.45) (end 192.309 88.49) (width 0.2) (layer "F.Cu") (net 11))
 (segment (start 170.949 87.45) (end 169.449 85.95) (width 0.2) (layer "F.Cu") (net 11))
 (segment (start 169.449 108.81) (end 170.5 107.759) (width 0.2) (layer "F.Cu") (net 11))
 (segment (start 170.5 107.759) (end 170.5 102.241) (width 0.2) (layer "F.Cu") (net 11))
 (segment (start 170.5 74.301) (end 169.449 73.25) (width 0.2) (layer "F.Cu") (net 11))
 (segment (start 199.949 116.83) (end 199.949 116.45) (width 0.2) (layer "F.Cu") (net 11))
 (segment (start 170.5 92.081) (end 169.449 91.03) (width 0.2) (layer "F.Cu") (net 11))
 (segment (start 170.5 102.241) (end 169.449 101.19) (width 0.2) (layer "F.Cu") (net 11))
 (segment (start 158.799 85.52) (end 169.019 85.52) (width 0.2) (layer "F.Cu") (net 11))
 (segment (start 194.349 78.83) (end 192.309 80.87) (width 0.2) (layer "F.Cu") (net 11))
 (segment (start 170.5 84.899) (end 170.5 74.301) (width 0.2) (layer "F.Cu") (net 11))
 (segment (start 170.949 89.53) (end 170.949 87.45) (width 0.2) (layer "F.Cu") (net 11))
 (segment (start 170.949 87.45) (end 191.269 87.45) (width 0.2) (layer "F.Cu") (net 11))
 (segment (start 169.449 101.19) (end 170.5 100.139) (width 0.2) (layer "F.Cu") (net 11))
 (segment (start 169.449 91.03) (end 170.949 89.53) (width 0.2) (layer "F.Cu") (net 11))
 (segment (start 169.449 85.95) (end 170.5 84.899) (width 0.2) (layer "F.Cu") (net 11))
 (segment (start 169.019 85.52) (end 169.449 85.95) (width 0.2) (layer "F.Cu") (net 11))
 (segment (start 199.949 116.45) (end 192.309 108.81) (width 0.2) (layer "F.Cu") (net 11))
 (segment (start 200.449 81.33) (end 199.949 81.33) (width 0.2) (layer "F.Cu") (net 11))
 (segment (start 194.449 78.83) (end 194.349 78.83) (width 0.2) (layer "F.Cu") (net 11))
 (segment (start 170.5 100.139) (end 170.5 92.081) (width 0.2) (layer "F.Cu") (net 11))
 (segment (start 199.949 81.33) (end 199.489 80.87) (width 0.2) (layer "F.Cu") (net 11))
 (segment (start 199.489 80.87) (end 192.309 80.87) (width 0.2) (layer "F.Cu") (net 11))
 (via (at 194.449 78.83) (size 0.6) (drill 0.3) (layers "F.Cu" "B.Cu") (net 11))
 (segment (start 192.309 80.87) (end 193.36 81.921) (width 0.2) (layer "B.Cu") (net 11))
 (segment (start 194.449 75.39) (end 194.449 78.83) (width 0.2) (layer "B.Cu") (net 11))
 (segment (start 192.309 88.49) (end 193.36 89.541) (width 0.2) (layer "B.Cu") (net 11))
 (segment (start 192.309 73.25) (end 194.449 75.39) (width 0.2) (layer "B.Cu") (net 11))
 (segment (start 192.309 101.19) (end 194.449 103.33) (width 0.2) (layer "B.Cu") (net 11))
 (segment (start 194.449 103.33) (end 194.449 106.67) (width 0.2) (layer "B.Cu") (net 11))
 (segment (start 193.36 81.921) (end 193.36 87.439) (width 0.2) (layer "B.Cu") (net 11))
 (segment (start 193.36 87.439) (end 192.309 88.49) (width 0.2) (layer "B.Cu") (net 11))
 (segment (start 194.449 106.67) (end 192.309 108.81) (width 0.2) (layer "B.Cu") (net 11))
 (segment (start 193.36 100.139) (end 192.309 101.19) (width 0.2) (layer "B.Cu") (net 11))
 (segment (start 193.36 89.541) (end 193.36 100.139) (width 0.2) (layer "B.Cu") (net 11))
 (segment (start 167.339 80.44) (end 169.449 78.33) (width 0.2) (layer "F.Cu") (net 13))
 (segment (start 169.449 75.79) (end 169.449 78.33) (width 0.2) (layer "F.Cu") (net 13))
 (segment (start 158.799 80.44) (end 167.339 80.44) (width 0.2) (layer "F.Cu") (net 13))
 (segment (start 200.449 78.79) (end 199.549 79.69) (width 0.2) (layer "B.Cu") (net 13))
 (segment (start 170.809 79.69) (end 169.449 78.33) (width 0.2) (layer "B.Cu") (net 13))
 (segment (start 199.549 79.69) (end 170.809 79.69) (width 0.2) (layer "B.Cu") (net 13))
 (segment (start 166.479 90.6) (end 169.449 93.57) (width 0.2) (layer "F.Cu") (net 33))
 (segment (start 158.799 90.6) (end 166.479 90.6) (width 0.2) (layer "F.Cu") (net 33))
 (segment (start 117 81.5) (end 117 78.2) (width 0.2) (layer "F.Cu") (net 24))
 (segment (start 97.71 89.5) (end 109 89.5) (width 0.2) (layer "F.Cu") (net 24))
 (segment (start 95.22 87.01) (end 97.71 89.5) (width 0.2) (layer "F.Cu") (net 24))
 (segment (start 109 89.5) (end 117 81.5) (width 0.2) (layer "F.Cu") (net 24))
 (segment (start 191.258 97.161) (end 191.258 101.625339) (width 0.2) (layer "F.Cu") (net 1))
 (segment (start 192.309 96.11) (end 191.258 97.161) (width 0.2) (layer "F.Cu") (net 1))
 (segment (start 192.271661 102.639) (end 192.758 102.639) (width 0.2) (layer "F.Cu") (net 1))
 (segment (start 192.758 102.639) (end 199.949 109.83) (width 0.2) (layer "F.Cu") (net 1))
 (segment (start 191.258 101.625339) (end 192.271661 102.639) (width 0.2) (layer "F.Cu") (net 1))
 (segment (start 199.949 109.83) (end 199.949 109.925) (width 0.2) (layer "F.Cu") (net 1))
 (segment (start 201.25 113.126) (end 201.25 120.029) (width 0.2) (layer "F.Cu") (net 2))
 (segment (start 201.25 120.029) (end 199.949 121.33) (width 0.2) (layer "F.Cu") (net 2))
 (segment (start 199.949 111.825) (end 201.25 113.126) (width 0.2) (layer "F.Cu") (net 2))
 (segment (start 97.46 78) (end 89.501 85.959) (width 0.2) (layer "B.Cu") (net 26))
 (segment (start 89.501 85.959) (end 83.571 85.959) (width 0.2) (layer "B.Cu") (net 26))
 (segment (start 83.571 85.959) (end 82.52 87.01) (width 0.2) (layer "B.Cu") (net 26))
 (segment (start 102.84 109.87) (end 105.38 109.87) (width 0.2) (layer "B.Cu") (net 20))
 (segment (start 70.92 79) (end 72.121 77.799) (width 0.2) (layer "F.Cu") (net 23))
 (segment (start 88.549 77.799) (end 97.76 87.01) (width 0.2) (layer "F.Cu") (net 23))
 (segment (start 72.121 77.799) (end 88.549 77.799) (width 0.2) (layer "F.Cu") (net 23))
 (segment (start 200.449 90.51) (end 192.309 98.65) (width 0.2) (layer "F.Cu") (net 12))
 (segment (start 200.449 83.87) (end 200.449 90.51) (width 0.2) (layer "F.Cu") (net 12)))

